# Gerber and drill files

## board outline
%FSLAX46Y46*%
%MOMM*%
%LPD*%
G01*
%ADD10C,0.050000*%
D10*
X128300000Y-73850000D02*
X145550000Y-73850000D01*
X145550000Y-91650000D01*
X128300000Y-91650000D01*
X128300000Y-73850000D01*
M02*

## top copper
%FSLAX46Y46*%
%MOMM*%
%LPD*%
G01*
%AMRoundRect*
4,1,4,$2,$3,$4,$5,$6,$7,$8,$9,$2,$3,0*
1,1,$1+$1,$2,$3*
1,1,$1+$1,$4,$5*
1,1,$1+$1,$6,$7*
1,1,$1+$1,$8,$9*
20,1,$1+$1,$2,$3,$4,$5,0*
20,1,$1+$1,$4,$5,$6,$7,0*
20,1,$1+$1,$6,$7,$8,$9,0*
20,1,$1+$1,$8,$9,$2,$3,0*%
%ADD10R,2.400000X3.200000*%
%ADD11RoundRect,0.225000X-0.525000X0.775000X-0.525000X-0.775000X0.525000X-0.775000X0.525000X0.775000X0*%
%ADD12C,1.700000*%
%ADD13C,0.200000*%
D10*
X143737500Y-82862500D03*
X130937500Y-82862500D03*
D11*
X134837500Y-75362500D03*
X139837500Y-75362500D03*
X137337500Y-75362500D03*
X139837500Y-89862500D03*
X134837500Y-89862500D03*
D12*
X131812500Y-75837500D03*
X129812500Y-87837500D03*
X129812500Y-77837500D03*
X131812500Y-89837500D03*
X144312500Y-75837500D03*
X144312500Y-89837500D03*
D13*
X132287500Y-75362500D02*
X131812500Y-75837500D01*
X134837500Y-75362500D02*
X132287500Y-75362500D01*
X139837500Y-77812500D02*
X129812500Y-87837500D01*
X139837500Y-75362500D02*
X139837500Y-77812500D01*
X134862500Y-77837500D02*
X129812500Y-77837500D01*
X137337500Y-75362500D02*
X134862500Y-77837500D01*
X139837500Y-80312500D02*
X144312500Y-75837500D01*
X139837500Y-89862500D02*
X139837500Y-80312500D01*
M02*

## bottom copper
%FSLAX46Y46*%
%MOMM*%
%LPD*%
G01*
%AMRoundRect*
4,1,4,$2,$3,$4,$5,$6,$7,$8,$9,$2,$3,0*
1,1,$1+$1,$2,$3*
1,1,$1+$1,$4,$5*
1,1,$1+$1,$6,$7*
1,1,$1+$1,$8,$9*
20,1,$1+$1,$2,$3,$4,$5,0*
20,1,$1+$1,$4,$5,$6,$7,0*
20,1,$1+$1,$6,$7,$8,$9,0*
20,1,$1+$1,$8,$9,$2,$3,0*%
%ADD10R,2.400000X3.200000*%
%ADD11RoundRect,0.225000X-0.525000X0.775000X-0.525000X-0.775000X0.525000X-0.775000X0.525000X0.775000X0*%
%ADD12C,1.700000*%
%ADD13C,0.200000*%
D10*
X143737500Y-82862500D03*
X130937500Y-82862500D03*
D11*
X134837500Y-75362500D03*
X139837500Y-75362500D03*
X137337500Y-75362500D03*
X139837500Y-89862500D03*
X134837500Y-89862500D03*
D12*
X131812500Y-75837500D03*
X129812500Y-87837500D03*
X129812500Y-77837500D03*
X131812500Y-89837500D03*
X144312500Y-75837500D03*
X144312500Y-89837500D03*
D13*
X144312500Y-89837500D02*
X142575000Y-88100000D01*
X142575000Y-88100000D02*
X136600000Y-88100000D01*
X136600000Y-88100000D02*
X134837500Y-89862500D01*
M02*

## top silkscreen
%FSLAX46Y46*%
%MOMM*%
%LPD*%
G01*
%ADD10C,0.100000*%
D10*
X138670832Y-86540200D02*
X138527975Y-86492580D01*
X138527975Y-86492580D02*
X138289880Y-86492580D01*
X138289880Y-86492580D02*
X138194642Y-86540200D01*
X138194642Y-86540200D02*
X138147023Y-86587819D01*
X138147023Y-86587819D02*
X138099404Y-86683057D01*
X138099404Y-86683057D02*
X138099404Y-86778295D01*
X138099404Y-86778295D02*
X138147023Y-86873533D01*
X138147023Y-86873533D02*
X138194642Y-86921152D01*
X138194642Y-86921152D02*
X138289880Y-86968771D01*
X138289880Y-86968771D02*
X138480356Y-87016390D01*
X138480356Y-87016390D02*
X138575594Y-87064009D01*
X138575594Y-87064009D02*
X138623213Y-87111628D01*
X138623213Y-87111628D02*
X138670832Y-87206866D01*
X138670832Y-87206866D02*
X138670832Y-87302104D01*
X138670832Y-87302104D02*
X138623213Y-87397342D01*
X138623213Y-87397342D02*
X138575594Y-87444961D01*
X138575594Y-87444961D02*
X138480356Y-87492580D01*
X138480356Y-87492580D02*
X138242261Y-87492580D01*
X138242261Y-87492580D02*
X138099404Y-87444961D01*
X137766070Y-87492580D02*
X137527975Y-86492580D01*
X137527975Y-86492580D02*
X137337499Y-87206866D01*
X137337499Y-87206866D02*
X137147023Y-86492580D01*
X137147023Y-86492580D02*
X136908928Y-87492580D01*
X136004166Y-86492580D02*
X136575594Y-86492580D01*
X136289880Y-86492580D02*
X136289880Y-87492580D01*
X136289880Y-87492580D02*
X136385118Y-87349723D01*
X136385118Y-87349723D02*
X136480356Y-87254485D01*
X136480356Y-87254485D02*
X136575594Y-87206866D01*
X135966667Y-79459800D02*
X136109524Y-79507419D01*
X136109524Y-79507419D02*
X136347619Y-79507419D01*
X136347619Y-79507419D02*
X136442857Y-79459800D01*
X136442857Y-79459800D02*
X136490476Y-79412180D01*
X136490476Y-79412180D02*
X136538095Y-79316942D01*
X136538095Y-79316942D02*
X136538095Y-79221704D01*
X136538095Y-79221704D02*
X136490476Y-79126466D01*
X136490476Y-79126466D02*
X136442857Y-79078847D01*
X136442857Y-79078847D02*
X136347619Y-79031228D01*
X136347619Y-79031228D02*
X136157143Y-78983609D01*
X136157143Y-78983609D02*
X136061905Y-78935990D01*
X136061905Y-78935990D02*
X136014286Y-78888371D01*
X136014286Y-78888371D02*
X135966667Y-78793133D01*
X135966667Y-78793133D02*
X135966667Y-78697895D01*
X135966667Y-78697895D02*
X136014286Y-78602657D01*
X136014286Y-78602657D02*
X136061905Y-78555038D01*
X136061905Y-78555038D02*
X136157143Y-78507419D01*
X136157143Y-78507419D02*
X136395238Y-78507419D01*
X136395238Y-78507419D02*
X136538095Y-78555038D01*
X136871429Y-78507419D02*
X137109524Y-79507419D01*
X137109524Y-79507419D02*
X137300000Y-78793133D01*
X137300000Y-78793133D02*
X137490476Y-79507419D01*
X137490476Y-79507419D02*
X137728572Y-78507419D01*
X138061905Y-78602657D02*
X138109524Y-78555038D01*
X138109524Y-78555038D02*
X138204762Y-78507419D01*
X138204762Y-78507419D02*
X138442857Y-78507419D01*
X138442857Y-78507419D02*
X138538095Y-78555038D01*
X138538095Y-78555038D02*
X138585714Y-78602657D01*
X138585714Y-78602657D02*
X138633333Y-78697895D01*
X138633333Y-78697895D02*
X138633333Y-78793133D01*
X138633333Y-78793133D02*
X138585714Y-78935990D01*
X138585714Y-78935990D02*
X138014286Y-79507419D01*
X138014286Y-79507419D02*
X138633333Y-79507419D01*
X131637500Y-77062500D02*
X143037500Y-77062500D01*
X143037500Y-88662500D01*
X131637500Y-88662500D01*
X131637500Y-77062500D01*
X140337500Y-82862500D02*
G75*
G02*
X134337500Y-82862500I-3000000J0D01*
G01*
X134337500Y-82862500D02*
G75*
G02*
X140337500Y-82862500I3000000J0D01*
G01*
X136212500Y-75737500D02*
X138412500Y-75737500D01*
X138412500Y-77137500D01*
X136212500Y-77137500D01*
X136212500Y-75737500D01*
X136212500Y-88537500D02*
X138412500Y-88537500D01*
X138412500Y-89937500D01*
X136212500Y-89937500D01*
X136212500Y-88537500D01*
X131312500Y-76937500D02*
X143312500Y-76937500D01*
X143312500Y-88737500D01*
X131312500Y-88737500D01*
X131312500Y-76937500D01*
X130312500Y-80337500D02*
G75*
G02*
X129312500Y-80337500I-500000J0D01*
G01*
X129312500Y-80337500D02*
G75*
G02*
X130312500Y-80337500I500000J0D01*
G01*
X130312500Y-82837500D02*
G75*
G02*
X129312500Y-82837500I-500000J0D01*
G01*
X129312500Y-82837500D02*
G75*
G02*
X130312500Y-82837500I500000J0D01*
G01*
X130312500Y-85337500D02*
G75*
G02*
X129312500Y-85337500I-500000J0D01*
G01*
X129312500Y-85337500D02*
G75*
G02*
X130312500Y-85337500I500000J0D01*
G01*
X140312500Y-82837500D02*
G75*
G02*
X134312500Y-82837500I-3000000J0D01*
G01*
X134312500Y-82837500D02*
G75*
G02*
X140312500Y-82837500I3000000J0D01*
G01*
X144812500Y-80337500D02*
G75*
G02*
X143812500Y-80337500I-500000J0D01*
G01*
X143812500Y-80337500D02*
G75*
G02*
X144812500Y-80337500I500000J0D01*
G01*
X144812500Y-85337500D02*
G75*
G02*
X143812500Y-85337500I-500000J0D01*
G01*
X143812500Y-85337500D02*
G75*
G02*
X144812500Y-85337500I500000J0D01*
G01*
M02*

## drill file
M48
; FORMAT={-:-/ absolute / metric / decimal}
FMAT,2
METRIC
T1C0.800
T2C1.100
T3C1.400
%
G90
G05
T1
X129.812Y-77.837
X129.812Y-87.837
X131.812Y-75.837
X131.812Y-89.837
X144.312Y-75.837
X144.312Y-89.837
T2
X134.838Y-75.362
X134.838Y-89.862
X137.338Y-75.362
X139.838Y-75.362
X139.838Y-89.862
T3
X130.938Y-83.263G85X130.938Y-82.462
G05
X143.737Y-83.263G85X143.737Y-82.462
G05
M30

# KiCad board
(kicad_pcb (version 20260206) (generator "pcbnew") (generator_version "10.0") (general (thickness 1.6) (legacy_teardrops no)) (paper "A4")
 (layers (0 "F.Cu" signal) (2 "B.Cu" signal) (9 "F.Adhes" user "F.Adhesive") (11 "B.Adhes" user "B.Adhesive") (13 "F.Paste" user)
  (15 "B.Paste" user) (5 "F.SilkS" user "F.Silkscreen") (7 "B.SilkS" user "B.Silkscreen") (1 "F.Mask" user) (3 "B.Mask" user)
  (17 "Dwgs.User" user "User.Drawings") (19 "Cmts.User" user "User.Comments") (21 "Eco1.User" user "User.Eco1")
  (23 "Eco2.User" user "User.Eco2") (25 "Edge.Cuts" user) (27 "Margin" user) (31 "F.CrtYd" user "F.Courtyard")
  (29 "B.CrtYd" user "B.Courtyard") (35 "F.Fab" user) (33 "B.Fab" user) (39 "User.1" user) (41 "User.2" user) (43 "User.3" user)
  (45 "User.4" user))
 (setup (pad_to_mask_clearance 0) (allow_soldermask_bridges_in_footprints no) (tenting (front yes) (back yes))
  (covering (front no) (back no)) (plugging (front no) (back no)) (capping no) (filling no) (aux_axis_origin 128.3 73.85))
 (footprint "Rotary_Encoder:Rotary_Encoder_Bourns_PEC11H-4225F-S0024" (layer "F.Cu") (at 137.3375 82.8625 180)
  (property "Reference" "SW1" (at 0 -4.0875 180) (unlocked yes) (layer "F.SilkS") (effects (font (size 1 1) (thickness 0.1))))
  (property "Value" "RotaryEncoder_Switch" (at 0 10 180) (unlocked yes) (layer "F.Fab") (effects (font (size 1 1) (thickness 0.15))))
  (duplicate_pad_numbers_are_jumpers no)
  (fp_rect (start -5.7 -5.8) (end 5.7 5.8) (stroke (width 0.1) (type default)) (fill no) (layer "F.SilkS"))
  (fp_circle (center 0 0) (end 3 0) (stroke (width 0.1) (type default)) (fill no) (layer "F.SilkS"))
  (pad "" np_thru_hole rect (at -6.4 0 180) (size 2.4 3.2) (drill oval 1.4 2.2) (layers "*.Cu" "*.Mask"))
  (pad "" np_thru_hole rect (at 6.4 0 180) (size 2.4 3.2) (drill oval 1.4 2.2) (layers "*.Cu" "*.Mask"))
  (pad "A" thru_hole roundrect (at 2.5 7.5 270) (size 2 1.5) (drill 1.1) (layers "*.Cu" "*.Mask") (remove_unused_layers no)
   (roundrect_rratio 0.15) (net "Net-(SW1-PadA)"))
  (pad "B" thru_hole roundrect (at -2.5 7.5 270) (size 2 1.5) (drill 1.1) (layers "*.Cu" "*.Mask") (remove_unused_layers no)
   (roundrect_rratio 0.15) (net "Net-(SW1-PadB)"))
  (pad "C" thru_hole roundrect (at 0 7.5 270) (size 2 1.5) (drill 1.1) (layers "*.Cu" "*.Mask") (remove_unused_layers no)
   (roundrect_rratio 0.15) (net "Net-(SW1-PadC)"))
  (pad "S1" thru_hole roundrect (at -2.5 -7 270) (size 2 1.5) (drill 1.1) (layers "*.Cu" "*.Mask") (remove_unused_layers no)
   (roundrect_rratio 0.15) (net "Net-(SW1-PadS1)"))
  (pad "S2" thru_hole roundrect (at 2.5 -7 270) (size 2 1.5) (drill 1.1) (layers "*.Cu" "*.Mask") (remove_unused_layers no)
   (roundrect_rratio 0.15) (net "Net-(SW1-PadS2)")))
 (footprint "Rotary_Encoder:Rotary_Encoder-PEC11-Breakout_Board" (layer "F.Cu") (at 137.3125 82.8375 -90)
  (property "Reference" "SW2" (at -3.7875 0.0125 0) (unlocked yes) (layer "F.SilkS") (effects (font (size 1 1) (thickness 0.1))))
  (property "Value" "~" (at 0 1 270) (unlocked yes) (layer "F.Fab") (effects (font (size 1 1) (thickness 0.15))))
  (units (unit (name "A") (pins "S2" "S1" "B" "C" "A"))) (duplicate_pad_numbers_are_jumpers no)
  (fp_rect (start -7.1 -1.1) (end -5.7 1.1) (stroke (width 0.1) (type default)) (fill no) (layer "F.SilkS"))
  (fp_rect (start 5.7 -1.1) (end 7.1 1.1) (stroke (width 0.1) (type default)) (fill no) (layer "F.SilkS"))
  (fp_rect (start -5.9 -6) (end 5.9 6) (stroke (width 0.1) (type default)) (fill no) (layer "F.SilkS"))
  (fp_circle (center -2.5 7.5) (end -2 7.5) (stroke (width 0.1) (type default)) (fill no) (layer "F.SilkS"))
  (fp_circle (center 0 7.5) (end 0.5 7.5) (stroke (width 0.1) (type default)) (fill no) (layer "F.SilkS"))
  (fp_circle (center 2.5 7.5) (end 3 7.5) (stroke (width 0.1) (type default)) (fill no) (layer "F.SilkS"))
  (fp_circle (center 0 0) (end 3 0) (stroke (width 0.1) (type default)) (fill no) (layer "F.SilkS"))
  (fp_circle (center -2.5 -7) (end -2 -7) (stroke (width 0.1) (type default)) (fill no) (layer "F.SilkS"))
  (fp_circle (center 2.5 -7) (end 3 -7) (stroke (width 0.1) (type default)) (fill no) (layer "F.SilkS"))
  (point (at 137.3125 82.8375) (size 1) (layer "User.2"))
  (pad "A" thru_hole circle (at -7 5.5 270) (size 1.7 1.7) (drill 0.8) (layers "*.Cu" "*.Mask") (remove_unused_layers no)
   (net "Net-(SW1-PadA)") (thermal_bridge_angle 90))
  (pad "B" thru_hole circle (at 5 7.5 270) (size 1.7 1.7) (drill 0.8) (layers "*.Cu" "*.Mask") (remove_unused_layers no)
   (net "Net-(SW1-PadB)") (thermal_bridge_angle 90))
  (pad "C" thru_hole circle (at -5 7.5 270) (size 1.7 1.7) (drill 0.8) (layers "*.Cu" "*.Mask") (remove_unused_layers no)
   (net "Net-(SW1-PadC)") (thermal_bridge_angle 90))
  (pad "NC" thru_hole circle (at 7 5.5 270) (size 1.7 1.7) (drill 0.8) (layers "*.Cu" "*.Mask") (remove_unused_layers no)
   (thermal_bridge_angle 90))
  (pad "S1" thru_hole circle (at -7 -7 270) (size 1.7 1.7) (drill 0.8) (layers "*.Cu" "*.Mask") (remove_unused_layers no)
   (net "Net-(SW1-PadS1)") (thermal_bridge_angle 90))
  (pad "S2" thru_hole circle (at 7 -7 270) (size 1.7 1.7) (drill 0.8) (layers "*.Cu" "*.Mask") (remove_unused_layers no)
   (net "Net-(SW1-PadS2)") (thermal_bridge_angle 90)))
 (gr_rect (start 128.3 73.85) (end 145.55 91.65) (stroke (width 0.05) (type default)) (fill no) (layer "Edge.Cuts"))
 (segment (start 132.2875 75.3625) (end 131.8125 75.8375) (width 0.2) (layer "F.Cu") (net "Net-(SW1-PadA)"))
 (segment (start 134.8375 75.3625) (end 132.2875 75.3625) (width 0.2) (layer "F.Cu") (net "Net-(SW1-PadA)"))
 (segment (start 139.8375 77.8125) (end 129.8125 87.8375) (width 0.2) (layer "F.Cu") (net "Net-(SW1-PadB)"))
 (segment (start 139.8375 75.3625) (end 139.8375 77.8125) (width 0.2) (layer "F.Cu") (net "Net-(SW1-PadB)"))
 (segment (start 134.8625 77.8375) (end 129.8125 77.8375) (width 0.2) (layer "F.Cu") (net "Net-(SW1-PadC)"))
 (segment (start 137.3375 75.3625) (end 134.8625 77.8375) (width 0.2) (layer "F.Cu") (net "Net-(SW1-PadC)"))
 (segment (start 139.8375 80.3125) (end 144.3125 75.8375) (width 0.2) (layer "F.Cu") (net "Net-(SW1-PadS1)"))
 (segment (start 139.8375 89.8625) (end 139.8375 80.3125) (width 0.2) (layer "F.Cu") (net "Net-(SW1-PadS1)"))
 (segment (start 144.3125 89.8375) (end 142.575 88.1) (width 0.2) (layer "B.Cu") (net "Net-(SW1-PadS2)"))
 (segment (start 142.575 88.1) (end 136.6 88.1) (width 0.2) (layer "B.Cu") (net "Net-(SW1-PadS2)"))
 (segment (start 136.6 88.1) (end 134.8375 89.8625) (width 0.2) (layer "B.Cu") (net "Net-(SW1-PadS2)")))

